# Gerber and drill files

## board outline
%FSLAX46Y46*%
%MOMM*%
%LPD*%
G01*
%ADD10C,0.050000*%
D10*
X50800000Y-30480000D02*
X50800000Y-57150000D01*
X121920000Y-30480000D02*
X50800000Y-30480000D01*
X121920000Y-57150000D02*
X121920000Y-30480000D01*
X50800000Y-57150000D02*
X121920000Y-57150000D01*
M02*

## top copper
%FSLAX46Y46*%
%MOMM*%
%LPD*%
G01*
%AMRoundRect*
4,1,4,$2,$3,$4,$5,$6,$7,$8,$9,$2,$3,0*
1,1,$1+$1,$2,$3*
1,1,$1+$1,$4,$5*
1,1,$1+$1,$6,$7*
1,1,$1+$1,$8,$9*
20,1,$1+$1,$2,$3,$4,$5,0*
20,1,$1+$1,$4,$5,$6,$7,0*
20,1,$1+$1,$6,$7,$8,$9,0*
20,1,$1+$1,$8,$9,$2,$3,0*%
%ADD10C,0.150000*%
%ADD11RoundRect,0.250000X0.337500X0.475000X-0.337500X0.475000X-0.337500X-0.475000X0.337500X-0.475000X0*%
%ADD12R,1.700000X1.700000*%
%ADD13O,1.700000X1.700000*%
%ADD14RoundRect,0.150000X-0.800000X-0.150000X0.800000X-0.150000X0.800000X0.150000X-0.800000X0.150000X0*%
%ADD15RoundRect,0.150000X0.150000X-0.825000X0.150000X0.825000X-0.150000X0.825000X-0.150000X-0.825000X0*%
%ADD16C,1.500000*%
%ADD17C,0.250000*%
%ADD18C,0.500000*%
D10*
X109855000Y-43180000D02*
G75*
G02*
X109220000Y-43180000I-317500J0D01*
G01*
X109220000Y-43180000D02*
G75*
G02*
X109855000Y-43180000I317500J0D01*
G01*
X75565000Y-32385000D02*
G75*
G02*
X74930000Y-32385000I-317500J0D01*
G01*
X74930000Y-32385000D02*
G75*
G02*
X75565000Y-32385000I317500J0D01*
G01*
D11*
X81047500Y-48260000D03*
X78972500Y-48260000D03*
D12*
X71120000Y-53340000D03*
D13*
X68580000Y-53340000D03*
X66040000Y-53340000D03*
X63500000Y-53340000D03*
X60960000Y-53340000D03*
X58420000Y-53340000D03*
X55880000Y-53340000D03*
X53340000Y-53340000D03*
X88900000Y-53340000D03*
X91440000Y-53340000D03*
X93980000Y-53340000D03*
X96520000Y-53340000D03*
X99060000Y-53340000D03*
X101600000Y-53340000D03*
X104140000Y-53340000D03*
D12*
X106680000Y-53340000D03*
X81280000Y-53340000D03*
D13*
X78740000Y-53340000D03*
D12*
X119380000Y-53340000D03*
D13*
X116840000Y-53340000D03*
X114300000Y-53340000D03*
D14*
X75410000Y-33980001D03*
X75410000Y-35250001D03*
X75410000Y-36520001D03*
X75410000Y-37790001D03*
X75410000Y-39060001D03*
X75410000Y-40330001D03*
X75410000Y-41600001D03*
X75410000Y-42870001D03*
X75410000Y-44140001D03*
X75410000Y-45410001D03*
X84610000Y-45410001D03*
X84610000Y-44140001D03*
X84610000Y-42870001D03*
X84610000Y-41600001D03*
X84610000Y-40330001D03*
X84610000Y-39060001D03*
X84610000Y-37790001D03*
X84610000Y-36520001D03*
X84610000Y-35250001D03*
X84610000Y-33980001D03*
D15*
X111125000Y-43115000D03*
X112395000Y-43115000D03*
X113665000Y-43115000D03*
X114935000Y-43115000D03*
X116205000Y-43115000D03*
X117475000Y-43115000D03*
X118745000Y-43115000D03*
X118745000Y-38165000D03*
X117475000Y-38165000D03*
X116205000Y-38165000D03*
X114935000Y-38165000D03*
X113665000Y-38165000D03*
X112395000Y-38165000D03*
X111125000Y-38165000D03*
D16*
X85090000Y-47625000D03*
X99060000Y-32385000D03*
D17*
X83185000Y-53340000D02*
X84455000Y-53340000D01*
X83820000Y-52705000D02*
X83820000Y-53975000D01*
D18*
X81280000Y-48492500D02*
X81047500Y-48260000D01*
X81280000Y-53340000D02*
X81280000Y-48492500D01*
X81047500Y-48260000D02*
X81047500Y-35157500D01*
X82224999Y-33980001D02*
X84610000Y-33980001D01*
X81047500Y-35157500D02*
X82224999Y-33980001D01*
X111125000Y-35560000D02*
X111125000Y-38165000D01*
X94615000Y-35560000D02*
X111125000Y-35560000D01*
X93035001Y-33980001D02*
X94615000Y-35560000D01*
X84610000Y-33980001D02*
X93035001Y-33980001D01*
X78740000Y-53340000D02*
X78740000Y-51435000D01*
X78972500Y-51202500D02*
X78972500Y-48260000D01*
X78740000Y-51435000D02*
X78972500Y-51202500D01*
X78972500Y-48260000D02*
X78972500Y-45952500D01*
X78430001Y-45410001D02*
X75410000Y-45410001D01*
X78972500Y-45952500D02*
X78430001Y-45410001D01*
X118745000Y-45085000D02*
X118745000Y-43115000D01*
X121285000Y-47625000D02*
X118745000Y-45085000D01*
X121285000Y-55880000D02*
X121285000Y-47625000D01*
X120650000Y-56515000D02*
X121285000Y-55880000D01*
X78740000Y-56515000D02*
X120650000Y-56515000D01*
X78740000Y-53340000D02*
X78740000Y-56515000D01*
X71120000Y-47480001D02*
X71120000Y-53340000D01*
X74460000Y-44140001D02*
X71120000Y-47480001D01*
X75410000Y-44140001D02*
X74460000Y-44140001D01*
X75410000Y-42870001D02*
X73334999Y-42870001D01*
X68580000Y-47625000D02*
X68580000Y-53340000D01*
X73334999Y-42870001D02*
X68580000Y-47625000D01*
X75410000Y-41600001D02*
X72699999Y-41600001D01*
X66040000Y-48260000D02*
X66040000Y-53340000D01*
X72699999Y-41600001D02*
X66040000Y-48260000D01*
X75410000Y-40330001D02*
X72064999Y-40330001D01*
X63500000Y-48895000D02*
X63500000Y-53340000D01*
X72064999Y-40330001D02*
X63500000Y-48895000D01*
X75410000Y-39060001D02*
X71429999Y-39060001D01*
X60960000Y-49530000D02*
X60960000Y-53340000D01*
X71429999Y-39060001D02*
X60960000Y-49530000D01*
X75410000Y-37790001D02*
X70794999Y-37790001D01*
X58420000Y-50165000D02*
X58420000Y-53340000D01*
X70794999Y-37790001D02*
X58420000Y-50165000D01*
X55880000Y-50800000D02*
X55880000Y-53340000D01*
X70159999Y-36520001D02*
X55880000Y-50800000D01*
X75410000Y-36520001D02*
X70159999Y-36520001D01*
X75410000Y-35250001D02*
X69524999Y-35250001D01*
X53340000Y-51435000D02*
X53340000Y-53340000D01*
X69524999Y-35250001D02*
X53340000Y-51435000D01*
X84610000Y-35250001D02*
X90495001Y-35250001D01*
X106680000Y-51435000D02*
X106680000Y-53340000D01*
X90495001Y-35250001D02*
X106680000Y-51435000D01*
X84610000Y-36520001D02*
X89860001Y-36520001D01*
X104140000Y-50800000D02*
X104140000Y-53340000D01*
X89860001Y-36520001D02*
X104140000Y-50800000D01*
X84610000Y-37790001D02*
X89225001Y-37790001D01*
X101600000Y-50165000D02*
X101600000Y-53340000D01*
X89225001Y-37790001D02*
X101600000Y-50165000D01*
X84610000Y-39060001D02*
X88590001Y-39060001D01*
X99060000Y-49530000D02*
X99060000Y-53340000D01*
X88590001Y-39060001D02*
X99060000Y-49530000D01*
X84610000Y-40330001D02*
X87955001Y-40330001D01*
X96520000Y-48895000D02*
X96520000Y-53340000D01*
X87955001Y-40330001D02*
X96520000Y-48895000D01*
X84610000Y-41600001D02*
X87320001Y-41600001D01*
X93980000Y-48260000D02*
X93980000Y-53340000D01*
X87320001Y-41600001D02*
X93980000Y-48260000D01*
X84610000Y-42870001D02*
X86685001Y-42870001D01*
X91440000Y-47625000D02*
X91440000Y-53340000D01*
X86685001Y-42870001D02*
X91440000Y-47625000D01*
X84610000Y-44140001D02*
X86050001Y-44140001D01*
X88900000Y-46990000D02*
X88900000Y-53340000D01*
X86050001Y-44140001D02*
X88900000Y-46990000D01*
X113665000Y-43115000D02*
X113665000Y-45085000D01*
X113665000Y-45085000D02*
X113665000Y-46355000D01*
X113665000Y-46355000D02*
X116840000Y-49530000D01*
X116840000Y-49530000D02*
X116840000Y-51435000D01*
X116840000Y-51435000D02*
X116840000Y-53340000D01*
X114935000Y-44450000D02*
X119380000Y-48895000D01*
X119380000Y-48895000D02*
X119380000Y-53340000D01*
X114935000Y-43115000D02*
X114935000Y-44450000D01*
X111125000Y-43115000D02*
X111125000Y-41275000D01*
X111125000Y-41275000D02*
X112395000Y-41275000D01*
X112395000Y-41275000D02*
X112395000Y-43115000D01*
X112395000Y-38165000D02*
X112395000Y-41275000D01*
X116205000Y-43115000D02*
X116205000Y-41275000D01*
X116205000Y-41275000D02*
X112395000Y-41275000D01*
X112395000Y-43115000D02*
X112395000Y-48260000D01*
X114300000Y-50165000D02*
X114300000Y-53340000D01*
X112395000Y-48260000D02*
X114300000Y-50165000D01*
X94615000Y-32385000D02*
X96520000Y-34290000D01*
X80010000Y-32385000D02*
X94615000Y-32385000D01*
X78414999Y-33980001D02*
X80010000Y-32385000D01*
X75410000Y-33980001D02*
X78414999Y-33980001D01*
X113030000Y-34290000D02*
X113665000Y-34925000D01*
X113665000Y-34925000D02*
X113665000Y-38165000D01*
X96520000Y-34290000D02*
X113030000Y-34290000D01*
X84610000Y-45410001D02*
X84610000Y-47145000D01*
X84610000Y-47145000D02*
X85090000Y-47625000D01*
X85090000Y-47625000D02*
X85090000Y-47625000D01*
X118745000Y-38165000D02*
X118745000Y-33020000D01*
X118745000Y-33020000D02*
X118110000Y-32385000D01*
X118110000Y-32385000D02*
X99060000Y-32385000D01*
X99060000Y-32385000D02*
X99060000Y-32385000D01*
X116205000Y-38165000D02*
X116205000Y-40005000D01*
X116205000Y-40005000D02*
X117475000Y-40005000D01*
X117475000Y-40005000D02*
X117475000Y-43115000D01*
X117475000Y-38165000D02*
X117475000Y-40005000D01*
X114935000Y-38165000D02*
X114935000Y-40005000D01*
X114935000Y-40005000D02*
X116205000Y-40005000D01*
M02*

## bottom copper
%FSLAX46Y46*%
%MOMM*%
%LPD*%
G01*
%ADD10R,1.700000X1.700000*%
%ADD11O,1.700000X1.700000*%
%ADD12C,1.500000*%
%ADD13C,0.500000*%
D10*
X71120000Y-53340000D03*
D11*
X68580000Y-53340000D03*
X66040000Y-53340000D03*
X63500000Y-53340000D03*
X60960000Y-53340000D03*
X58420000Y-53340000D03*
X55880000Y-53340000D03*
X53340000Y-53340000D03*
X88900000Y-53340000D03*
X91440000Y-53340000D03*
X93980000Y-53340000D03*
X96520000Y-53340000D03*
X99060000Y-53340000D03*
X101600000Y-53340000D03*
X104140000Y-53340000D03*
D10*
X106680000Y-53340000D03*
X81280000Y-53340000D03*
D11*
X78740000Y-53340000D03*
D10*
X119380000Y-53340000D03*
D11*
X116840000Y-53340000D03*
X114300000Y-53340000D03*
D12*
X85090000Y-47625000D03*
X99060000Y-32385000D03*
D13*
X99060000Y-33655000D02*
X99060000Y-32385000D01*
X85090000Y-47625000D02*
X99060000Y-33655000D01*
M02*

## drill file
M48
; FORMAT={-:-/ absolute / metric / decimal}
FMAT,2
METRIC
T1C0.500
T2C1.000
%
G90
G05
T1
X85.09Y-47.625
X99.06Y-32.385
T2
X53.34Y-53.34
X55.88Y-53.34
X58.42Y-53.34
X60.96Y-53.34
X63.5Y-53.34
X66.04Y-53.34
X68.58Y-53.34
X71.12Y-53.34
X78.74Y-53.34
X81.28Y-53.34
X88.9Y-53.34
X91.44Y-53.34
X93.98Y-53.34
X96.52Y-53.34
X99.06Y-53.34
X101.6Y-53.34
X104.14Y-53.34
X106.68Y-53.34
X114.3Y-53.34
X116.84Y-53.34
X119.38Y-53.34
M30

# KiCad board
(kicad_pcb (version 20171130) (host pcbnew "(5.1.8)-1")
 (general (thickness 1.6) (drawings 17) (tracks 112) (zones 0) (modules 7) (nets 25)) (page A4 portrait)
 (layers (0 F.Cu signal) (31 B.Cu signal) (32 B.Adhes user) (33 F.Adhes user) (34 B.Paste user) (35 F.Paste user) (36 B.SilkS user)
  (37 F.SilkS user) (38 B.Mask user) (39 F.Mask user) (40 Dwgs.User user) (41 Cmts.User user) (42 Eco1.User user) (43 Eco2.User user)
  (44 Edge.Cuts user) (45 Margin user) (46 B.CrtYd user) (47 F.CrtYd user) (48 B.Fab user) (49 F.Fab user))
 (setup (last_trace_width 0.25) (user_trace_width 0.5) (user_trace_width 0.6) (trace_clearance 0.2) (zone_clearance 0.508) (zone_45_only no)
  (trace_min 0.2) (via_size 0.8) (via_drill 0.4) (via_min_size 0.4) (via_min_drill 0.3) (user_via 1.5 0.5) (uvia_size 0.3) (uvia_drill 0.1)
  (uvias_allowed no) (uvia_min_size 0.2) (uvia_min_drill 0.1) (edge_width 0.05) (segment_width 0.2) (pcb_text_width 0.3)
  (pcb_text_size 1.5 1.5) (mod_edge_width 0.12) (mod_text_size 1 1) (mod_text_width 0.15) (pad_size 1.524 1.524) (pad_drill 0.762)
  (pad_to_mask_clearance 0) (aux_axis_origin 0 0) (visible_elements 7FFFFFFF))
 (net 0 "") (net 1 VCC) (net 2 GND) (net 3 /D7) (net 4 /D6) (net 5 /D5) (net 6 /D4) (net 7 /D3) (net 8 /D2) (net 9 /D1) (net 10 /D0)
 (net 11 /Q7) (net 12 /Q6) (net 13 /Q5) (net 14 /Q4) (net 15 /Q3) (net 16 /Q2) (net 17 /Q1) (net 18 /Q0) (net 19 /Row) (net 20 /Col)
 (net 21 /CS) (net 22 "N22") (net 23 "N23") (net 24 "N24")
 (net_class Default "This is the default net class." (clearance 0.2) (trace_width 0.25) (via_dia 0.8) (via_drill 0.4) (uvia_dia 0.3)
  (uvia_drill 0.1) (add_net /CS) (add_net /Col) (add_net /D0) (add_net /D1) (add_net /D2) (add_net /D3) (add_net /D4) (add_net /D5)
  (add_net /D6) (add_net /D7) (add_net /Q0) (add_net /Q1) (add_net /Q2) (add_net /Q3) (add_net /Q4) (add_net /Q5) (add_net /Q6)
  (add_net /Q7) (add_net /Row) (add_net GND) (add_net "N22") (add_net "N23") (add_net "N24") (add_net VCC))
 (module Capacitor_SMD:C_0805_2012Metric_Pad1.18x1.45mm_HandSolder (layer F.Cu) (at 80.01 48.26 180)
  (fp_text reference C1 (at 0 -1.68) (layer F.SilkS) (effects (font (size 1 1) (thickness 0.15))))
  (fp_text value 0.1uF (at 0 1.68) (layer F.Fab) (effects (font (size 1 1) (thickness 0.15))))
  (pad 1 smd roundrect (at -1.0375 0 180) (size 1.175 1.45) (layers F.Cu F.Paste F.Mask) (roundrect_rratio 0.212766) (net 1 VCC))
  (pad 2 smd roundrect (at 1.0375 0 180) (size 1.175 1.45) (layers F.Cu F.Paste F.Mask) (roundrect_rratio 0.212766) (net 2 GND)))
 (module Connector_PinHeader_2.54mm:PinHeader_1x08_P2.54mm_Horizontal (layer F.Cu) (at 71.12 53.34 270)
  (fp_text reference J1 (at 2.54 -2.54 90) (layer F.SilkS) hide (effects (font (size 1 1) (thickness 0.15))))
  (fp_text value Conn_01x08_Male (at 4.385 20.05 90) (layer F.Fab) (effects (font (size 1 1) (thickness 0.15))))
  (pad 1 thru_hole rect (at 0 0 270) (size 1.7 1.7) (drill 1) (layers *.Cu *.Mask) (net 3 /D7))
  (pad 2 thru_hole oval (at 0 2.54 270) (size 1.7 1.7) (drill 1) (layers *.Cu *.Mask) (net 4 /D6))
  (pad 3 thru_hole oval (at 0 5.08 270) (size 1.7 1.7) (drill 1) (layers *.Cu *.Mask) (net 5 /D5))
  (pad 4 thru_hole oval (at 0 7.62 270) (size 1.7 1.7) (drill 1) (layers *.Cu *.Mask) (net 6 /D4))
  (pad 5 thru_hole oval (at 0 10.16 270) (size 1.7 1.7) (drill 1) (layers *.Cu *.Mask) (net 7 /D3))
  (pad 6 thru_hole oval (at 0 12.7 270) (size 1.7 1.7) (drill 1) (layers *.Cu *.Mask) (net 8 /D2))
  (pad 7 thru_hole oval (at 0 15.24 270) (size 1.7 1.7) (drill 1) (layers *.Cu *.Mask) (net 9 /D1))
  (pad 8 thru_hole oval (at 0 17.78 270) (size 1.7 1.7) (drill 1) (layers *.Cu *.Mask) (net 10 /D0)))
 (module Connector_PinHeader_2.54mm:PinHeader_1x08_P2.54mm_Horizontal (layer F.Cu) (at 106.68 53.34 270)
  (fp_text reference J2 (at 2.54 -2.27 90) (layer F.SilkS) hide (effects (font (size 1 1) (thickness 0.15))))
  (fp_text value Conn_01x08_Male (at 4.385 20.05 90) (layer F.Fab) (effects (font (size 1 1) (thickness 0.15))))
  (pad 8 thru_hole oval (at 0 17.78 270) (size 1.7 1.7) (drill 1) (layers *.Cu *.Mask) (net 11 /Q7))
  (pad 7 thru_hole oval (at 0 15.24 270) (size 1.7 1.7) (drill 1) (layers *.Cu *.Mask) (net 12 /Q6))
  (pad 6 thru_hole oval (at 0 12.7 270) (size 1.7 1.7) (drill 1) (layers *.Cu *.Mask) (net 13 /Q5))
  (pad 5 thru_hole oval (at 0 10.16 270) (size 1.7 1.7) (drill 1) (layers *.Cu *.Mask) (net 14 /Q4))
  (pad 4 thru_hole oval (at 0 7.62 270) (size 1.7 1.7) (drill 1) (layers *.Cu *.Mask) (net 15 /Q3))
  (pad 3 thru_hole oval (at 0 5.08 270) (size 1.7 1.7) (drill 1) (layers *.Cu *.Mask) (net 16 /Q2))
  (pad 2 thru_hole oval (at 0 2.54 270) (size 1.7 1.7) (drill 1) (layers *.Cu *.Mask) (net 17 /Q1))
  (pad 1 thru_hole rect (at 0 0 270) (size 1.7 1.7) (drill 1) (layers *.Cu *.Mask) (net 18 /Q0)))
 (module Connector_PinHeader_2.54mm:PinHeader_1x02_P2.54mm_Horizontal (layer F.Cu) (at 81.28 53.34 270)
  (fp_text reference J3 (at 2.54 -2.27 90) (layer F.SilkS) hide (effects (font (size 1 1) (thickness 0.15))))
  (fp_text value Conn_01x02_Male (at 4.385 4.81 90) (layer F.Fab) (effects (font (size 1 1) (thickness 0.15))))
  (pad 1 thru_hole rect (at 0 0 270) (size 1.7 1.7) (drill 1) (layers *.Cu *.Mask) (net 1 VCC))
  (pad 2 thru_hole oval (at 0 2.54 270) (size 1.7 1.7) (drill 1) (layers *.Cu *.Mask) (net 2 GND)))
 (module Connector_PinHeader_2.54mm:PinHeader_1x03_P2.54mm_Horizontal (layer F.Cu) (at 119.38 53.34 270)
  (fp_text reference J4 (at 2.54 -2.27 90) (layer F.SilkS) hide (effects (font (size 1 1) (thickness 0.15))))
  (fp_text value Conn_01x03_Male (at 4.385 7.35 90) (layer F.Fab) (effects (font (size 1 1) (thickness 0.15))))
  (pad 1 thru_hole rect (at 0 0 270) (size 1.7 1.7) (drill 1) (layers *.Cu *.Mask) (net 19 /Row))
  (pad 2 thru_hole oval (at 0 2.54 270) (size 1.7 1.7) (drill 1) (layers *.Cu *.Mask) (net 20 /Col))
  (pad 3 thru_hole oval (at 0 5.08 270) (size 1.7 1.7) (drill 1) (layers *.Cu *.Mask) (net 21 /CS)))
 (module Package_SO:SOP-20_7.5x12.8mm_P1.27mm (layer F.Cu) (at 80.01 39.695001)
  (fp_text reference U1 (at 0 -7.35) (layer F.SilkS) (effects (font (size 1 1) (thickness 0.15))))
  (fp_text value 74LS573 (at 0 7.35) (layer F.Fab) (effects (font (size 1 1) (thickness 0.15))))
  (pad 1 smd roundrect (at -4.6 -5.715) (size 1.9 0.6) (layers F.Cu F.Paste F.Mask) (roundrect_rratio 0.25) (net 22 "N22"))
  (pad 2 smd roundrect (at -4.6 -4.445) (size 1.9 0.6) (layers F.Cu F.Paste F.Mask) (roundrect_rratio 0.25) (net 10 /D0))
  (pad 3 smd roundrect (at -4.6 -3.175) (size 1.9 0.6) (layers F.Cu F.Paste F.Mask) (roundrect_rratio 0.25) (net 9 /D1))
  (pad 4 smd roundrect (at -4.6 -1.905) (size 1.9 0.6) (layers F.Cu F.Paste F.Mask) (roundrect_rratio 0.25) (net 8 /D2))
  (pad 5 smd roundrect (at -4.6 -0.635) (size 1.9 0.6) (layers F.Cu F.Paste F.Mask) (roundrect_rratio 0.25) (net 7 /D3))
  (pad 6 smd roundrect (at -4.6 0.635) (size 1.9 0.6) (layers F.Cu F.Paste F.Mask) (roundrect_rratio 0.25) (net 6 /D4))
  (pad 7 smd roundrect (at -4.6 1.905) (size 1.9 0.6) (layers F.Cu F.Paste F.Mask) (roundrect_rratio 0.25) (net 5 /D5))
  (pad 8 smd roundrect (at -4.6 3.175) (size 1.9 0.6) (layers F.Cu F.Paste F.Mask) (roundrect_rratio 0.25) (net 4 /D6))
  (pad 9 smd roundrect (at -4.6 4.445) (size 1.9 0.6) (layers F.Cu F.Paste F.Mask) (roundrect_rratio 0.25) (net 3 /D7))
  (pad 10 smd roundrect (at -4.6 5.715) (size 1.9 0.6) (layers F.Cu F.Paste F.Mask) (roundrect_rratio 0.25) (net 2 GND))
  (pad 11 smd roundrect (at 4.6 5.715) (size 1.9 0.6) (layers F.Cu F.Paste F.Mask) (roundrect_rratio 0.25) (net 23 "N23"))
  (pad 12 smd roundrect (at 4.6 4.445) (size 1.9 0.6) (layers F.Cu F.Paste F.Mask) (roundrect_rratio 0.25) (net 11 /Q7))
  (pad 13 smd roundrect (at 4.6 3.175) (size 1.9 0.6) (layers F.Cu F.Paste F.Mask) (roundrect_rratio 0.25) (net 12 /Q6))
  (pad 14 smd roundrect (at 4.6 1.905) (size 1.9 0.6) (layers F.Cu F.Paste F.Mask) (roundrect_rratio 0.25) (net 13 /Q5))
  (pad 15 smd roundrect (at 4.6 0.635) (size 1.9 0.6) (layers F.Cu F.Paste F.Mask) (roundrect_rratio 0.25) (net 14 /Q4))
  (pad 16 smd roundrect (at 4.6 -0.635) (size 1.9 0.6) (layers F.Cu F.Paste F.Mask) (roundrect_rratio 0.25) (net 15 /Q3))
  (pad 17 smd roundrect (at 4.6 -1.905) (size 1.9 0.6) (layers F.Cu F.Paste F.Mask) (roundrect_rratio 0.25) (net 16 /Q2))
  (pad 18 smd roundrect (at 4.6 -3.175) (size 1.9 0.6) (layers F.Cu F.Paste F.Mask) (roundrect_rratio 0.25) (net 17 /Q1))
  (pad 19 smd roundrect (at 4.6 -4.445) (size 1.9 0.6) (layers F.Cu F.Paste F.Mask) (roundrect_rratio 0.25) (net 18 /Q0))
  (pad 20 smd roundrect (at 4.6 -5.715) (size 1.9 0.6) (layers F.Cu F.Paste F.Mask) (roundrect_rratio 0.25) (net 1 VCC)))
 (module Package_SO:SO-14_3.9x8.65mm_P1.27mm (layer F.Cu) (at 114.935 40.64 90)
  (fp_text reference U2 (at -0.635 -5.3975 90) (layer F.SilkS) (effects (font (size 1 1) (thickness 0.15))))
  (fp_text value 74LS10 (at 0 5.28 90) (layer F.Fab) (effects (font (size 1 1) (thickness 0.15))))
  (pad 1 smd roundrect (at -2.475 -3.81 90) (size 1.95 0.6) (layers F.Cu F.Paste F.Mask) (roundrect_rratio 0.25) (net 21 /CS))
  (pad 2 smd roundrect (at -2.475 -2.54 90) (size 1.95 0.6) (layers F.Cu F.Paste F.Mask) (roundrect_rratio 0.25) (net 21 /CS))
  (pad 3 smd roundrect (at -2.475 -1.27 90) (size 1.95 0.6) (layers F.Cu F.Paste F.Mask) (roundrect_rratio 0.25) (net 20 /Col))
  (pad 4 smd roundrect (at -2.475 0 90) (size 1.95 0.6) (layers F.Cu F.Paste F.Mask) (roundrect_rratio 0.25) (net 19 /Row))
  (pad 5 smd roundrect (at -2.475 1.27 90) (size 1.95 0.6) (layers F.Cu F.Paste F.Mask) (roundrect_rratio 0.25) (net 21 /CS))
  (pad 6 smd roundrect (at -2.475 2.54 90) (size 1.95 0.6) (layers F.Cu F.Paste F.Mask) (roundrect_rratio 0.25) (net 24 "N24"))
  (pad 7 smd roundrect (at -2.475 3.81 90) (size 1.95 0.6) (layers F.Cu F.Paste F.Mask) (roundrect_rratio 0.25) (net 2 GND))
  (pad 8 smd roundrect (at 2.475 3.81 90) (size 1.95 0.6) (layers F.Cu F.Paste F.Mask) (roundrect_rratio 0.25) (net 23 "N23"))
  (pad 9 smd roundrect (at 2.475 2.54 90) (size 1.95 0.6) (layers F.Cu F.Paste F.Mask) (roundrect_rratio 0.25) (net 24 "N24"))
  (pad 10 smd roundrect (at 2.475 1.27 90) (size 1.95 0.6) (layers F.Cu F.Paste F.Mask) (roundrect_rratio 0.25) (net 24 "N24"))
  (pad 11 smd roundrect (at 2.475 0 90) (size 1.95 0.6) (layers F.Cu F.Paste F.Mask) (roundrect_rratio 0.25) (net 24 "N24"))
  (pad 12 smd roundrect (at 2.475 -1.27 90) (size 1.95 0.6) (layers F.Cu F.Paste F.Mask) (roundrect_rratio 0.25) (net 22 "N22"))
  (pad 13 smd roundrect (at 2.475 -2.54 90) (size 1.95 0.6) (layers F.Cu F.Paste F.Mask) (roundrect_rratio 0.25) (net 21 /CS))
  (pad 14 smd roundrect (at 2.475 -3.81 90) (size 1.95 0.6) (layers F.Cu F.Paste F.Mask) (roundrect_rratio 0.25) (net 1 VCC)))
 (gr_circle (center 109.5375 43.18) (end 109.855 43.18) (layer F.Cu) (width 0.15))
 (gr_circle (center 75.2475 32.385) (end 75.565 32.385) (layer F.Cu) (width 0.15))
 (gr_line (start 50.8 30.48) (end 50.8 57.15) (layer Edge.Cuts) (width 0.05))
 (gr_line (start 121.92 30.48) (end 50.8 30.48) (layer Edge.Cuts) (width 0.05))
 (gr_line (start 121.92 57.15) (end 121.92 30.48) (layer Edge.Cuts) (width 0.05))
 (gr_line (start 50.8 57.15) (end 121.92 57.15) (layer Edge.Cuts) (width 0.05))
 (segment (start 83.185 53.34) (end 84.455 53.34) (width 0.25) (layer F.Cu) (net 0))
 (segment (start 83.82 52.705) (end 83.82 53.975) (width 0.25) (layer F.Cu) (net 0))
 (segment (start 81.28 48.4925) (end 81.0475 48.26) (width 0.5) (layer F.Cu) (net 1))
 (segment (start 81.28 53.34) (end 81.28 48.4925) (width 0.5) (layer F.Cu) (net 1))
 (segment (start 81.0475 48.26) (end 81.0475 35.1575) (width 0.5) (layer F.Cu) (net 1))
 (segment (start 82.224999 33.980001) (end 84.61 33.980001) (width 0.5) (layer F.Cu) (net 1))
 (segment (start 81.0475 35.1575) (end 82.224999 33.980001) (width 0.5) (layer F.Cu) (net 1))
 (segment (start 111.125 35.56) (end 111.125 38.165) (width 0.5) (layer F.Cu) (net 1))
 (segment (start 94.615 35.56) (end 111.125 35.56) (width 0.5) (layer F.Cu) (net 1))
 (segment (start 93.035001 33.980001) (end 94.615 35.56) (width 0.5) (layer F.Cu) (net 1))
 (segment (start 84.61 33.980001) (end 93.035001 33.980001) (width 0.5) (layer F.Cu) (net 1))
 (segment (start 78.74 53.34) (end 78.74 51.435) (width 0.5) (layer F.Cu) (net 2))
 (segment (start 78.9725 51.2025) (end 78.9725 48.26) (width 0.5) (layer F.Cu) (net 2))
 (segment (start 78.74 51.435) (end 78.9725 51.2025) (width 0.5) (layer F.Cu) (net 2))
 (segment (start 78.9725 48.26) (end 78.9725 45.9525) (width 0.5) (layer F.Cu) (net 2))
 (segment (start 78.430001 45.410001) (end 75.41 45.410001) (width 0.5) (layer F.Cu) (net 2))
 (segment (start 78.9725 45.9525) (end 78.430001 45.410001) (width 0.5) (layer F.Cu) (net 2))
 (segment (start 118.745 45.085) (end 118.745 43.115) (width 0.5) (layer F.Cu) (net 2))
 (segment (start 121.285 47.625) (end 118.745 45.085) (width 0.5) (layer F.Cu) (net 2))
 (segment (start 121.285 55.88) (end 121.285 47.625) (width 0.5) (layer F.Cu) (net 2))
 (segment (start 120.65 56.515) (end 121.285 55.88) (width 0.5) (layer F.Cu) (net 2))
 (segment (start 78.74 56.515) (end 120.65 56.515) (width 0.5) (layer F.Cu) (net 2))
 (segment (start 78.74 53.34) (end 78.74 56.515) (width 0.5) (layer F.Cu) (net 2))
 (segment (start 71.12 47.480001) (end 71.12 53.34) (width 0.5) (layer F.Cu) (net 3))
 (segment (start 74.46 44.140001) (end 71.12 47.480001) (width 0.5) (layer F.Cu) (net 3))
 (segment (start 75.41 44.140001) (end 74.46 44.140001) (width 0.5) (layer F.Cu) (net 3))
 (segment (start 75.41 42.870001) (end 73.334999 42.870001) (width 0.5) (layer F.Cu) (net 4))
 (segment (start 68.58 47.625) (end 68.58 53.34) (width 0.5) (layer F.Cu) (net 4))
 (segment (start 73.334999 42.870001) (end 68.58 47.625) (width 0.5) (layer F.Cu) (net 4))
 (segment (start 75.41 41.600001) (end 72.699999 41.600001) (width 0.5) (layer F.Cu) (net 5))
 (segment (start 66.04 48.26) (end 66.04 53.34) (width 0.5) (layer F.Cu) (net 5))
 (segment (start 72.699999 41.600001) (end 66.04 48.26) (width 0.5) (layer F.Cu) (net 5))
 (segment (start 75.41 40.330001) (end 72.064999 40.330001) (width 0.5) (layer F.Cu) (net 6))
 (segment (start 63.5 48.895) (end 63.5 53.34) (width 0.5) (layer F.Cu) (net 6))
 (segment (start 72.064999 40.330001) (end 63.5 48.895) (width 0.5) (layer F.Cu) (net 6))
 (segment (start 75.41 39.060001) (end 71.429999 39.060001) (width 0.5) (layer F.Cu) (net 7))
 (segment (start 60.96 49.53) (end 60.96 53.34) (width 0.5) (layer F.Cu) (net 7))
 (segment (start 71.429999 39.060001) (end 60.96 49.53) (width 0.5) (layer F.Cu) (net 7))
 (segment (start 75.41 37.790001) (end 70.794999 37.790001) (width 0.5) (layer F.Cu) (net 8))
 (segment (start 58.42 50.165) (end 58.42 53.34) (width 0.5) (layer F.Cu) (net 8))
 (segment (start 70.794999 37.790001) (end 58.42 50.165) (width 0.5) (layer F.Cu) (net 8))
 (segment (start 55.88 50.8) (end 55.88 53.34) (width 0.5) (layer F.Cu) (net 9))
 (segment (start 70.159999 36.520001) (end 55.88 50.8) (width 0.5) (layer F.Cu) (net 9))
 (segment (start 75.41 36.520001) (end 70.159999 36.520001) (width 0.5) (layer F.Cu) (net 9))
 (segment (start 75.41 35.250001) (end 69.524999 35.250001) (width 0.5) (layer F.Cu) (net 10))
 (segment (start 53.34 51.435) (end 53.34 53.34) (width 0.5) (layer F.Cu) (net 10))
 (segment (start 69.524999 35.250001) (end 53.34 51.435) (width 0.5) (layer F.Cu) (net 10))
 (segment (start 84.61 35.250001) (end 90.495001 35.250001) (width 0.5) (layer F.Cu) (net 18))
 (segment (start 106.68 51.435) (end 106.68 53.34) (width 0.5) (layer F.Cu) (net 18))
 (segment (start 90.495001 35.250001) (end 106.68 51.435) (width 0.5) (layer F.Cu) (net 18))
 (segment (start 84.61 36.520001) (end 89.860001 36.520001) (width 0.5) (layer F.Cu) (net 17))
 (segment (start 104.14 50.8) (end 104.14 53.34) (width 0.5) (layer F.Cu) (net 17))
 (segment (start 89.860001 36.520001) (end 104.14 50.8) (width 0.5) (layer F.Cu) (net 17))
 (segment (start 84.61 37.790001) (end 89.225001 37.790001) (width 0.5) (layer F.Cu) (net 16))
 (segment (start 101.6 50.165) (end 101.6 53.34) (width 0.5) (layer F.Cu) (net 16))
 (segment (start 89.225001 37.790001) (end 101.6 50.165) (width 0.5) (layer F.Cu) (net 16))
 (segment (start 84.61 39.060001) (end 88.590001 39.060001) (width 0.5) (layer F.Cu) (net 15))
 (segment (start 99.06 49.53) (end 99.06 53.34) (width 0.5) (layer F.Cu) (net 15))
 (segment (start 88.590001 39.060001) (end 99.06 49.53) (width 0.5) (layer F.Cu) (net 15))
 (segment (start 84.61 40.330001) (end 87.955001 40.330001) (width 0.5) (layer F.Cu) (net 14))
 (segment (start 96.52 48.895) (end 96.52 53.34) (width 0.5) (layer F.Cu) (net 14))
 (segment (start 87.955001 40.330001) (end 96.52 48.895) (width 0.5) (layer F.Cu) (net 14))
 (segment (start 84.61 41.600001) (end 87.320001 41.600001) (width 0.5) (layer F.Cu) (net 13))
 (segment (start 93.98 48.26) (end 93.98 53.34) (width 0.5) (layer F.Cu) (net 13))
 (segment (start 87.320001 41.600001) (end 93.98 48.26) (width 0.5) (layer F.Cu) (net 13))
 (segment (start 84.61 42.870001) (end 86.685001 42.870001) (width 0.5) (layer F.Cu) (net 12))
 (segment (start 91.44 47.625) (end 91.44 53.34) (width 0.5) (layer F.Cu) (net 12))
 (segment (start 86.685001 42.870001) (end 91.44 47.625) (width 0.5) (layer F.Cu) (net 12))
 (segment (start 84.61 44.140001) (end 86.050001 44.140001) (width 0.5) (layer F.Cu) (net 11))
 (segment (start 88.9 46.99) (end 88.9 53.34) (width 0.5) (layer F.Cu) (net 11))
 (segment (start 86.050001 44.140001) (end 88.9 46.99) (width 0.5) (layer F.Cu) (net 11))
 (segment (start 113.665 43.115) (end 113.665 45.085) (width 0.5) (layer F.Cu) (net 20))
 (segment (start 113.665 45.085) (end 113.665 46.355) (width 0.5) (layer F.Cu) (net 20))
 (segment (start 113.665 46.355) (end 116.84 49.53) (width 0.5) (layer F.Cu) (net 20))
 (segment (start 116.84 49.53) (end 116.84 51.435) (width 0.5) (layer F.Cu) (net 20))
 (segment (start 116.84 51.435) (end 116.84 53.34) (width 0.5) (layer F.Cu) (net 20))
 (segment (start 114.935 44.45) (end 119.38 48.895) (width 0.5) (layer F.Cu) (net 19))
 (segment (start 119.38 48.895) (end 119.38 53.34) (width 0.5) (layer F.Cu) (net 19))
 (segment (start 114.935 43.115) (end 114.935 44.45) (width 0.5) (layer F.Cu) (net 19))
 (segment (start 111.125 43.115) (end 111.125 41.275) (width 0.5) (layer F.Cu) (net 21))
 (segment (start 111.125 41.275) (end 112.395 41.275) (width 0.5) (layer F.Cu) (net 21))
 (segment (start 112.395 41.275) (end 112.395 43.115) (width 0.5) (layer F.Cu) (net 21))
 (segment (start 112.395 38.165) (end 112.395 41.275) (width 0.5) (layer F.Cu) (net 21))
 (segment (start 116.205 43.115) (end 116.205 41.275) (width 0.5) (layer F.Cu) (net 21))
 (segment (start 116.205 41.275) (end 112.395 41.275) (width 0.5) (layer F.Cu) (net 21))
 (segment (start 112.395 43.115) (end 112.395 48.26) (width 0.5) (layer F.Cu) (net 21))
 (segment (start 114.3 50.165) (end 114.3 53.34) (width 0.5) (layer F.Cu) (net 21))
 (segment (start 112.395 48.26) (end 114.3 50.165) (width 0.5) (layer F.Cu) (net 21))
 (segment (start 94.615 32.385) (end 96.52 34.29) (width 0.5) (layer F.Cu) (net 22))
 (segment (start 80.01 32.385) (end 94.615 32.385) (width 0.5) (layer F.Cu) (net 22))
 (segment (start 78.414999 33.980001) (end 80.01 32.385) (width 0.5) (layer F.Cu) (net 22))
 (segment (start 75.41 33.980001) (end 78.414999 33.980001) (width 0.5) (layer F.Cu) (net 22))
 (segment (start 113.03 34.29) (end 113.665 34.925) (width 0.5) (layer F.Cu) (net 22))
 (segment (start 113.665 34.925) (end 113.665 38.165) (width 0.5) (layer F.Cu) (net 22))
 (segment (start 96.52 34.29) (end 113.03 34.29) (width 0.5) (layer F.Cu) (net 22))
 (segment (start 84.61 45.410001) (end 84.61 47.145) (width 0.5) (layer F.Cu) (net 23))
 (segment (start 84.61 47.145) (end 85.09 47.625) (width 0.5) (layer F.Cu) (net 23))
 (segment (start 85.09 47.625) (end 85.09 47.625) (width 0.5) (layer F.Cu) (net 23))
 (via (at 85.09 47.625) (size 1.5) (drill 0.5) (layers F.Cu B.Cu) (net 23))
 (segment (start 118.745 38.165) (end 118.745 33.02) (width 0.5) (layer F.Cu) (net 23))
 (segment (start 118.745 33.02) (end 118.11 32.385) (width 0.5) (layer F.Cu) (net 23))
 (segment (start 118.11 32.385) (end 99.06 32.385) (width 0.5) (layer F.Cu) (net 23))
 (segment (start 99.06 32.385) (end 99.06 32.385) (width 0.5) (layer F.Cu) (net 23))
 (via (at 99.06 32.385) (size 1.5) (drill 0.5) (layers F.Cu B.Cu) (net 23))
 (segment (start 99.06 33.655) (end 99.06 32.385) (width 0.5) (layer B.Cu) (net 23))
 (segment (start 85.09 47.625) (end 99.06 33.655) (width 0.5) (layer B.Cu) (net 23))
 (segment (start 116.205 38.165) (end 116.205 40.005) (width 0.5) (layer F.Cu) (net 24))
 (segment (start 116.205 40.005) (end 117.475 40.005) (width 0.5) (layer F.Cu) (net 24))
 (segment (start 117.475 40.005) (end 117.475 43.115) (width 0.5) (layer F.Cu) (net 24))
 (segment (start 117.475 38.165) (end 117.475 40.005) (width 0.5) (layer F.Cu) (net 24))
 (segment (start 114.935 38.165) (end 114.935 40.005) (width 0.5) (layer F.Cu) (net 24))
 (segment (start 114.935 40.005) (end 116.205 40.005) (width 0.5) (layer F.Cu) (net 24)))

